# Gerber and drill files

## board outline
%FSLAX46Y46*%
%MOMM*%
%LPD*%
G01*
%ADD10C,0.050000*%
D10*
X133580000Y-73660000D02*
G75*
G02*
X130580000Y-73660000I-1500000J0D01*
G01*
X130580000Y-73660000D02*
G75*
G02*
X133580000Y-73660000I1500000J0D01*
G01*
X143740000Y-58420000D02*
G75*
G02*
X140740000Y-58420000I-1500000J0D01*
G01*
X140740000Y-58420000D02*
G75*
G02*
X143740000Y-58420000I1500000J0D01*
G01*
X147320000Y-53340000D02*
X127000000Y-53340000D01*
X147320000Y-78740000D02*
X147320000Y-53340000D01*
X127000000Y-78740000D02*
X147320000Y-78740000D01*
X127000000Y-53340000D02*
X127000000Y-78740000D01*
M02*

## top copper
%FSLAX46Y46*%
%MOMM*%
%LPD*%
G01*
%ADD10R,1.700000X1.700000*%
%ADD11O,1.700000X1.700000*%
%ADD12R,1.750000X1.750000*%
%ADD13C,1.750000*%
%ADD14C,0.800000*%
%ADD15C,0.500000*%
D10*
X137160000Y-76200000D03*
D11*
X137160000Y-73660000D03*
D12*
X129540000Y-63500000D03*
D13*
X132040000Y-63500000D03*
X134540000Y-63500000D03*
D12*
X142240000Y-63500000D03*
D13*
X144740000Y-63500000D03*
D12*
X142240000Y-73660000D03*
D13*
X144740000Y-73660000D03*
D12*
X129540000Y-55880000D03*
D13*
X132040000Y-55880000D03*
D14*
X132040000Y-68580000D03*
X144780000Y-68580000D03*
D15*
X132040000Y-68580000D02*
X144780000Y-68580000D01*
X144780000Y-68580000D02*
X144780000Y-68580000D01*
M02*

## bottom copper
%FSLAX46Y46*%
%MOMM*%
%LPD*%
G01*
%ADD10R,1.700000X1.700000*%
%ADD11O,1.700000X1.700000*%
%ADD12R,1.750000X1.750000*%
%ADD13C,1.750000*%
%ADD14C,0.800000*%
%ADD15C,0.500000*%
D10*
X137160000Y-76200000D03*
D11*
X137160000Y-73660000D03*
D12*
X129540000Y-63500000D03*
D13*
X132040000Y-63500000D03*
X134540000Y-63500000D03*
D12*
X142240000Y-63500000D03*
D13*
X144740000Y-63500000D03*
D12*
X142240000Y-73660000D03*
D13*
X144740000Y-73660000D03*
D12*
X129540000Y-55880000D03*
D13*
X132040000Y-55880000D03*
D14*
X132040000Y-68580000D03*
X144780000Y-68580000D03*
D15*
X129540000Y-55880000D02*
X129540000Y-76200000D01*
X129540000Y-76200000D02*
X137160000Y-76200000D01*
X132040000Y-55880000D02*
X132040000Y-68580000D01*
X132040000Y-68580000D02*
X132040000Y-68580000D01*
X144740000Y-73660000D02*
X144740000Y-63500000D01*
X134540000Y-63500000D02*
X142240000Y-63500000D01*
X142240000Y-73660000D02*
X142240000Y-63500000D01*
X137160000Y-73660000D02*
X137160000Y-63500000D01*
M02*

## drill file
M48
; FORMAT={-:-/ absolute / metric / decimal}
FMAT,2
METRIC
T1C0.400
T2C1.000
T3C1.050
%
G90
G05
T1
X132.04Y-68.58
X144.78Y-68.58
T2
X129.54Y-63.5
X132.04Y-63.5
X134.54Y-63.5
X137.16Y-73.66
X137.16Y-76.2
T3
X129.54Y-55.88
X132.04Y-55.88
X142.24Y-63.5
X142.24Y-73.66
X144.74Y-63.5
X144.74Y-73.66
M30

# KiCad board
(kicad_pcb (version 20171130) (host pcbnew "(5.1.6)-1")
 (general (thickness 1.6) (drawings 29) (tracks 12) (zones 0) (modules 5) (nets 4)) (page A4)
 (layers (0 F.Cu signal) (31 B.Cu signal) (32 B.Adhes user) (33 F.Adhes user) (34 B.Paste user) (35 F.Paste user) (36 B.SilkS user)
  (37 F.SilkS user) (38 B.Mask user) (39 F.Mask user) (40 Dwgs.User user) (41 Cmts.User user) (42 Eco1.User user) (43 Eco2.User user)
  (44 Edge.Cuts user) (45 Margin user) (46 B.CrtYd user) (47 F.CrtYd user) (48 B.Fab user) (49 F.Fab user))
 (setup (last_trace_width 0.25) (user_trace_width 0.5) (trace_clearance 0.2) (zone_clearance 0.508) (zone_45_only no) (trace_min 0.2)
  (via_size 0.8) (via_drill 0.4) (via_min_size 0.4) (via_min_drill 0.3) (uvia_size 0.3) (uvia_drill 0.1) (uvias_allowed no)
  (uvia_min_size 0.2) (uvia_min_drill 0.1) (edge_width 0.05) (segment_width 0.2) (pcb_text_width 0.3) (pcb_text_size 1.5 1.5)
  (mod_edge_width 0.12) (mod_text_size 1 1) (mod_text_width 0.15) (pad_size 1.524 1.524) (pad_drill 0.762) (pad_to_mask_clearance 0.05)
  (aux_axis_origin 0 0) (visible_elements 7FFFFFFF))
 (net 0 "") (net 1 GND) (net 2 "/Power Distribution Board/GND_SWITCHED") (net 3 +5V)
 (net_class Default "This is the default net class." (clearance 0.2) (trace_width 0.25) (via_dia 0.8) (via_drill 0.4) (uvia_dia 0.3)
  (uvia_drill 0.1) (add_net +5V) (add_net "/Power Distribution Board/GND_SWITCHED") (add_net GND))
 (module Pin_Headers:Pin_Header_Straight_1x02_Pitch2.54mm (layer F.Cu) (at 137.16 76.2 180)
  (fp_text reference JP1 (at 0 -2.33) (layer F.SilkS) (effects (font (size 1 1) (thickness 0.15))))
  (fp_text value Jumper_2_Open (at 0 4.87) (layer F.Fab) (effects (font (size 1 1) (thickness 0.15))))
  (pad 1 thru_hole rect (at 0 0 180) (size 1.7 1.7) (drill 1) (layers *.Cu *.Mask) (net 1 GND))
  (pad 2 thru_hole oval (at 0 2.54 180) (size 1.7 1.7) (drill 1) (layers *.Cu *.Mask) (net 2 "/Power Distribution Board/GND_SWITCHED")))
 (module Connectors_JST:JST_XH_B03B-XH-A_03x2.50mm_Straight (layer F.Cu) (at 129.54 63.5)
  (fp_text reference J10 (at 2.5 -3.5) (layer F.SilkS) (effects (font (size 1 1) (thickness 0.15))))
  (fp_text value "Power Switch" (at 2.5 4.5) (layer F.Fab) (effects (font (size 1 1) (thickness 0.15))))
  (pad 1 thru_hole rect (at 0 0) (size 1.75 1.75) (drill 1) (layers *.Cu *.Mask) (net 1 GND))
  (pad 2 thru_hole circle (at 2.5 0) (size 1.75 1.75) (drill 1) (layers *.Cu *.Mask) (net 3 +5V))
  (pad 3 thru_hole circle (at 5 0) (size 1.75 1.75) (drill 1) (layers *.Cu *.Mask) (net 2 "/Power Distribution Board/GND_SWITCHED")))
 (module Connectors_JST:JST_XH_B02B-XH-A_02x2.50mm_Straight (layer F.Cu) (at 142.24 63.5)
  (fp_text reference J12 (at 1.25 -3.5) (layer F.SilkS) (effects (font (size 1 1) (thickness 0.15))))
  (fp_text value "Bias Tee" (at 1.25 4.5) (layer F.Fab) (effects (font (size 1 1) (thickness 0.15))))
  (pad 1 thru_hole rect (at 0 0) (size 1.75 1.75) (drill 1.05) (layers *.Cu *.Mask) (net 2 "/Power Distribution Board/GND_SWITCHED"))
  (pad 2 thru_hole circle (at 2.5 0) (size 1.75 1.75) (drill 1.05) (layers *.Cu *.Mask) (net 3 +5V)))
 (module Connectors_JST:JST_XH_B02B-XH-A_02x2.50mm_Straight (layer F.Cu) (at 142.24 73.66)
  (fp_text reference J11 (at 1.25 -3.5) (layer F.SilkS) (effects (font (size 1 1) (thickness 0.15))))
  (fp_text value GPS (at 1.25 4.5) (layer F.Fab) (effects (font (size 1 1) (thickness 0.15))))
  (pad 1 thru_hole rect (at 0 0) (size 1.75 1.75) (drill 1.05) (layers *.Cu *.Mask) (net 2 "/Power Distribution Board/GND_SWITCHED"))
  (pad 2 thru_hole circle (at 2.5 0) (size 1.75 1.75) (drill 1.05) (layers *.Cu *.Mask) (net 3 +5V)))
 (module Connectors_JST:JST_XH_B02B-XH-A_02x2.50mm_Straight (layer F.Cu) (at 129.54 55.88)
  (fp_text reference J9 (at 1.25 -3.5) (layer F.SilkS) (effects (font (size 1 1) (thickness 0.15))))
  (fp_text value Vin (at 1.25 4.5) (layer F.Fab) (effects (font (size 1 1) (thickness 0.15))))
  (pad 1 thru_hole rect (at 0 0) (size 1.75 1.75) (drill 1.05) (layers *.Cu *.Mask) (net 1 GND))
  (pad 2 thru_hole circle (at 2.5 0) (size 1.75 1.75) (drill 1.05) (layers *.Cu *.Mask) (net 3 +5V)))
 (gr_circle (center 132.08 73.66) (end 133.58 73.66) (layer Edge.Cuts) (width 0.05))
 (gr_circle (center 142.24 58.42) (end 143.74 58.42) (layer Edge.Cuts) (width 0.05))
 (gr_line (start 147.32 53.34) (end 127 53.34) (layer Edge.Cuts) (width 0.05))
 (gr_line (start 147.32 78.74) (end 147.32 53.34) (layer Edge.Cuts) (width 0.05))
 (gr_line (start 127 78.74) (end 147.32 78.74) (layer Edge.Cuts) (width 0.05))
 (gr_line (start 127 53.34) (end 127 78.74) (layer Edge.Cuts) (width 0.05))
 (segment (start 129.54 55.88) (end 129.54 76.2) (width 0.5) (layer B.Cu) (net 1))
 (segment (start 129.54 76.2) (end 137.16 76.2) (width 0.5) (layer B.Cu) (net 1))
 (segment (start 132.04 55.88) (end 132.04 68.58) (width 0.5) (layer B.Cu) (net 3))
 (segment (start 132.04 68.58) (end 132.04 68.58) (width 0.5) (layer B.Cu) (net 3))
 (via (at 132.04 68.58) (size 0.8) (drill 0.4) (layers F.Cu B.Cu) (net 3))
 (segment (start 132.04 68.58) (end 144.78 68.58) (width 0.5) (layer F.Cu) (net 3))
 (segment (start 144.78 68.58) (end 144.78 68.58) (width 0.5) (layer F.Cu) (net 3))
 (via (at 144.78 68.58) (size 0.8) (drill 0.4) (layers F.Cu B.Cu) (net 3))
 (segment (start 144.74 73.66) (end 144.74 63.5) (width 0.5) (layer B.Cu) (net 3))
 (segment (start 134.54 63.5) (end 142.24 63.5) (width 0.5) (layer B.Cu) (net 2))
 (segment (start 142.24 73.66) (end 142.24 63.5) (width 0.5) (layer B.Cu) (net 2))
 (segment (start 137.16 73.66) (end 137.16 63.5) (width 0.5) (layer B.Cu) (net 2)))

